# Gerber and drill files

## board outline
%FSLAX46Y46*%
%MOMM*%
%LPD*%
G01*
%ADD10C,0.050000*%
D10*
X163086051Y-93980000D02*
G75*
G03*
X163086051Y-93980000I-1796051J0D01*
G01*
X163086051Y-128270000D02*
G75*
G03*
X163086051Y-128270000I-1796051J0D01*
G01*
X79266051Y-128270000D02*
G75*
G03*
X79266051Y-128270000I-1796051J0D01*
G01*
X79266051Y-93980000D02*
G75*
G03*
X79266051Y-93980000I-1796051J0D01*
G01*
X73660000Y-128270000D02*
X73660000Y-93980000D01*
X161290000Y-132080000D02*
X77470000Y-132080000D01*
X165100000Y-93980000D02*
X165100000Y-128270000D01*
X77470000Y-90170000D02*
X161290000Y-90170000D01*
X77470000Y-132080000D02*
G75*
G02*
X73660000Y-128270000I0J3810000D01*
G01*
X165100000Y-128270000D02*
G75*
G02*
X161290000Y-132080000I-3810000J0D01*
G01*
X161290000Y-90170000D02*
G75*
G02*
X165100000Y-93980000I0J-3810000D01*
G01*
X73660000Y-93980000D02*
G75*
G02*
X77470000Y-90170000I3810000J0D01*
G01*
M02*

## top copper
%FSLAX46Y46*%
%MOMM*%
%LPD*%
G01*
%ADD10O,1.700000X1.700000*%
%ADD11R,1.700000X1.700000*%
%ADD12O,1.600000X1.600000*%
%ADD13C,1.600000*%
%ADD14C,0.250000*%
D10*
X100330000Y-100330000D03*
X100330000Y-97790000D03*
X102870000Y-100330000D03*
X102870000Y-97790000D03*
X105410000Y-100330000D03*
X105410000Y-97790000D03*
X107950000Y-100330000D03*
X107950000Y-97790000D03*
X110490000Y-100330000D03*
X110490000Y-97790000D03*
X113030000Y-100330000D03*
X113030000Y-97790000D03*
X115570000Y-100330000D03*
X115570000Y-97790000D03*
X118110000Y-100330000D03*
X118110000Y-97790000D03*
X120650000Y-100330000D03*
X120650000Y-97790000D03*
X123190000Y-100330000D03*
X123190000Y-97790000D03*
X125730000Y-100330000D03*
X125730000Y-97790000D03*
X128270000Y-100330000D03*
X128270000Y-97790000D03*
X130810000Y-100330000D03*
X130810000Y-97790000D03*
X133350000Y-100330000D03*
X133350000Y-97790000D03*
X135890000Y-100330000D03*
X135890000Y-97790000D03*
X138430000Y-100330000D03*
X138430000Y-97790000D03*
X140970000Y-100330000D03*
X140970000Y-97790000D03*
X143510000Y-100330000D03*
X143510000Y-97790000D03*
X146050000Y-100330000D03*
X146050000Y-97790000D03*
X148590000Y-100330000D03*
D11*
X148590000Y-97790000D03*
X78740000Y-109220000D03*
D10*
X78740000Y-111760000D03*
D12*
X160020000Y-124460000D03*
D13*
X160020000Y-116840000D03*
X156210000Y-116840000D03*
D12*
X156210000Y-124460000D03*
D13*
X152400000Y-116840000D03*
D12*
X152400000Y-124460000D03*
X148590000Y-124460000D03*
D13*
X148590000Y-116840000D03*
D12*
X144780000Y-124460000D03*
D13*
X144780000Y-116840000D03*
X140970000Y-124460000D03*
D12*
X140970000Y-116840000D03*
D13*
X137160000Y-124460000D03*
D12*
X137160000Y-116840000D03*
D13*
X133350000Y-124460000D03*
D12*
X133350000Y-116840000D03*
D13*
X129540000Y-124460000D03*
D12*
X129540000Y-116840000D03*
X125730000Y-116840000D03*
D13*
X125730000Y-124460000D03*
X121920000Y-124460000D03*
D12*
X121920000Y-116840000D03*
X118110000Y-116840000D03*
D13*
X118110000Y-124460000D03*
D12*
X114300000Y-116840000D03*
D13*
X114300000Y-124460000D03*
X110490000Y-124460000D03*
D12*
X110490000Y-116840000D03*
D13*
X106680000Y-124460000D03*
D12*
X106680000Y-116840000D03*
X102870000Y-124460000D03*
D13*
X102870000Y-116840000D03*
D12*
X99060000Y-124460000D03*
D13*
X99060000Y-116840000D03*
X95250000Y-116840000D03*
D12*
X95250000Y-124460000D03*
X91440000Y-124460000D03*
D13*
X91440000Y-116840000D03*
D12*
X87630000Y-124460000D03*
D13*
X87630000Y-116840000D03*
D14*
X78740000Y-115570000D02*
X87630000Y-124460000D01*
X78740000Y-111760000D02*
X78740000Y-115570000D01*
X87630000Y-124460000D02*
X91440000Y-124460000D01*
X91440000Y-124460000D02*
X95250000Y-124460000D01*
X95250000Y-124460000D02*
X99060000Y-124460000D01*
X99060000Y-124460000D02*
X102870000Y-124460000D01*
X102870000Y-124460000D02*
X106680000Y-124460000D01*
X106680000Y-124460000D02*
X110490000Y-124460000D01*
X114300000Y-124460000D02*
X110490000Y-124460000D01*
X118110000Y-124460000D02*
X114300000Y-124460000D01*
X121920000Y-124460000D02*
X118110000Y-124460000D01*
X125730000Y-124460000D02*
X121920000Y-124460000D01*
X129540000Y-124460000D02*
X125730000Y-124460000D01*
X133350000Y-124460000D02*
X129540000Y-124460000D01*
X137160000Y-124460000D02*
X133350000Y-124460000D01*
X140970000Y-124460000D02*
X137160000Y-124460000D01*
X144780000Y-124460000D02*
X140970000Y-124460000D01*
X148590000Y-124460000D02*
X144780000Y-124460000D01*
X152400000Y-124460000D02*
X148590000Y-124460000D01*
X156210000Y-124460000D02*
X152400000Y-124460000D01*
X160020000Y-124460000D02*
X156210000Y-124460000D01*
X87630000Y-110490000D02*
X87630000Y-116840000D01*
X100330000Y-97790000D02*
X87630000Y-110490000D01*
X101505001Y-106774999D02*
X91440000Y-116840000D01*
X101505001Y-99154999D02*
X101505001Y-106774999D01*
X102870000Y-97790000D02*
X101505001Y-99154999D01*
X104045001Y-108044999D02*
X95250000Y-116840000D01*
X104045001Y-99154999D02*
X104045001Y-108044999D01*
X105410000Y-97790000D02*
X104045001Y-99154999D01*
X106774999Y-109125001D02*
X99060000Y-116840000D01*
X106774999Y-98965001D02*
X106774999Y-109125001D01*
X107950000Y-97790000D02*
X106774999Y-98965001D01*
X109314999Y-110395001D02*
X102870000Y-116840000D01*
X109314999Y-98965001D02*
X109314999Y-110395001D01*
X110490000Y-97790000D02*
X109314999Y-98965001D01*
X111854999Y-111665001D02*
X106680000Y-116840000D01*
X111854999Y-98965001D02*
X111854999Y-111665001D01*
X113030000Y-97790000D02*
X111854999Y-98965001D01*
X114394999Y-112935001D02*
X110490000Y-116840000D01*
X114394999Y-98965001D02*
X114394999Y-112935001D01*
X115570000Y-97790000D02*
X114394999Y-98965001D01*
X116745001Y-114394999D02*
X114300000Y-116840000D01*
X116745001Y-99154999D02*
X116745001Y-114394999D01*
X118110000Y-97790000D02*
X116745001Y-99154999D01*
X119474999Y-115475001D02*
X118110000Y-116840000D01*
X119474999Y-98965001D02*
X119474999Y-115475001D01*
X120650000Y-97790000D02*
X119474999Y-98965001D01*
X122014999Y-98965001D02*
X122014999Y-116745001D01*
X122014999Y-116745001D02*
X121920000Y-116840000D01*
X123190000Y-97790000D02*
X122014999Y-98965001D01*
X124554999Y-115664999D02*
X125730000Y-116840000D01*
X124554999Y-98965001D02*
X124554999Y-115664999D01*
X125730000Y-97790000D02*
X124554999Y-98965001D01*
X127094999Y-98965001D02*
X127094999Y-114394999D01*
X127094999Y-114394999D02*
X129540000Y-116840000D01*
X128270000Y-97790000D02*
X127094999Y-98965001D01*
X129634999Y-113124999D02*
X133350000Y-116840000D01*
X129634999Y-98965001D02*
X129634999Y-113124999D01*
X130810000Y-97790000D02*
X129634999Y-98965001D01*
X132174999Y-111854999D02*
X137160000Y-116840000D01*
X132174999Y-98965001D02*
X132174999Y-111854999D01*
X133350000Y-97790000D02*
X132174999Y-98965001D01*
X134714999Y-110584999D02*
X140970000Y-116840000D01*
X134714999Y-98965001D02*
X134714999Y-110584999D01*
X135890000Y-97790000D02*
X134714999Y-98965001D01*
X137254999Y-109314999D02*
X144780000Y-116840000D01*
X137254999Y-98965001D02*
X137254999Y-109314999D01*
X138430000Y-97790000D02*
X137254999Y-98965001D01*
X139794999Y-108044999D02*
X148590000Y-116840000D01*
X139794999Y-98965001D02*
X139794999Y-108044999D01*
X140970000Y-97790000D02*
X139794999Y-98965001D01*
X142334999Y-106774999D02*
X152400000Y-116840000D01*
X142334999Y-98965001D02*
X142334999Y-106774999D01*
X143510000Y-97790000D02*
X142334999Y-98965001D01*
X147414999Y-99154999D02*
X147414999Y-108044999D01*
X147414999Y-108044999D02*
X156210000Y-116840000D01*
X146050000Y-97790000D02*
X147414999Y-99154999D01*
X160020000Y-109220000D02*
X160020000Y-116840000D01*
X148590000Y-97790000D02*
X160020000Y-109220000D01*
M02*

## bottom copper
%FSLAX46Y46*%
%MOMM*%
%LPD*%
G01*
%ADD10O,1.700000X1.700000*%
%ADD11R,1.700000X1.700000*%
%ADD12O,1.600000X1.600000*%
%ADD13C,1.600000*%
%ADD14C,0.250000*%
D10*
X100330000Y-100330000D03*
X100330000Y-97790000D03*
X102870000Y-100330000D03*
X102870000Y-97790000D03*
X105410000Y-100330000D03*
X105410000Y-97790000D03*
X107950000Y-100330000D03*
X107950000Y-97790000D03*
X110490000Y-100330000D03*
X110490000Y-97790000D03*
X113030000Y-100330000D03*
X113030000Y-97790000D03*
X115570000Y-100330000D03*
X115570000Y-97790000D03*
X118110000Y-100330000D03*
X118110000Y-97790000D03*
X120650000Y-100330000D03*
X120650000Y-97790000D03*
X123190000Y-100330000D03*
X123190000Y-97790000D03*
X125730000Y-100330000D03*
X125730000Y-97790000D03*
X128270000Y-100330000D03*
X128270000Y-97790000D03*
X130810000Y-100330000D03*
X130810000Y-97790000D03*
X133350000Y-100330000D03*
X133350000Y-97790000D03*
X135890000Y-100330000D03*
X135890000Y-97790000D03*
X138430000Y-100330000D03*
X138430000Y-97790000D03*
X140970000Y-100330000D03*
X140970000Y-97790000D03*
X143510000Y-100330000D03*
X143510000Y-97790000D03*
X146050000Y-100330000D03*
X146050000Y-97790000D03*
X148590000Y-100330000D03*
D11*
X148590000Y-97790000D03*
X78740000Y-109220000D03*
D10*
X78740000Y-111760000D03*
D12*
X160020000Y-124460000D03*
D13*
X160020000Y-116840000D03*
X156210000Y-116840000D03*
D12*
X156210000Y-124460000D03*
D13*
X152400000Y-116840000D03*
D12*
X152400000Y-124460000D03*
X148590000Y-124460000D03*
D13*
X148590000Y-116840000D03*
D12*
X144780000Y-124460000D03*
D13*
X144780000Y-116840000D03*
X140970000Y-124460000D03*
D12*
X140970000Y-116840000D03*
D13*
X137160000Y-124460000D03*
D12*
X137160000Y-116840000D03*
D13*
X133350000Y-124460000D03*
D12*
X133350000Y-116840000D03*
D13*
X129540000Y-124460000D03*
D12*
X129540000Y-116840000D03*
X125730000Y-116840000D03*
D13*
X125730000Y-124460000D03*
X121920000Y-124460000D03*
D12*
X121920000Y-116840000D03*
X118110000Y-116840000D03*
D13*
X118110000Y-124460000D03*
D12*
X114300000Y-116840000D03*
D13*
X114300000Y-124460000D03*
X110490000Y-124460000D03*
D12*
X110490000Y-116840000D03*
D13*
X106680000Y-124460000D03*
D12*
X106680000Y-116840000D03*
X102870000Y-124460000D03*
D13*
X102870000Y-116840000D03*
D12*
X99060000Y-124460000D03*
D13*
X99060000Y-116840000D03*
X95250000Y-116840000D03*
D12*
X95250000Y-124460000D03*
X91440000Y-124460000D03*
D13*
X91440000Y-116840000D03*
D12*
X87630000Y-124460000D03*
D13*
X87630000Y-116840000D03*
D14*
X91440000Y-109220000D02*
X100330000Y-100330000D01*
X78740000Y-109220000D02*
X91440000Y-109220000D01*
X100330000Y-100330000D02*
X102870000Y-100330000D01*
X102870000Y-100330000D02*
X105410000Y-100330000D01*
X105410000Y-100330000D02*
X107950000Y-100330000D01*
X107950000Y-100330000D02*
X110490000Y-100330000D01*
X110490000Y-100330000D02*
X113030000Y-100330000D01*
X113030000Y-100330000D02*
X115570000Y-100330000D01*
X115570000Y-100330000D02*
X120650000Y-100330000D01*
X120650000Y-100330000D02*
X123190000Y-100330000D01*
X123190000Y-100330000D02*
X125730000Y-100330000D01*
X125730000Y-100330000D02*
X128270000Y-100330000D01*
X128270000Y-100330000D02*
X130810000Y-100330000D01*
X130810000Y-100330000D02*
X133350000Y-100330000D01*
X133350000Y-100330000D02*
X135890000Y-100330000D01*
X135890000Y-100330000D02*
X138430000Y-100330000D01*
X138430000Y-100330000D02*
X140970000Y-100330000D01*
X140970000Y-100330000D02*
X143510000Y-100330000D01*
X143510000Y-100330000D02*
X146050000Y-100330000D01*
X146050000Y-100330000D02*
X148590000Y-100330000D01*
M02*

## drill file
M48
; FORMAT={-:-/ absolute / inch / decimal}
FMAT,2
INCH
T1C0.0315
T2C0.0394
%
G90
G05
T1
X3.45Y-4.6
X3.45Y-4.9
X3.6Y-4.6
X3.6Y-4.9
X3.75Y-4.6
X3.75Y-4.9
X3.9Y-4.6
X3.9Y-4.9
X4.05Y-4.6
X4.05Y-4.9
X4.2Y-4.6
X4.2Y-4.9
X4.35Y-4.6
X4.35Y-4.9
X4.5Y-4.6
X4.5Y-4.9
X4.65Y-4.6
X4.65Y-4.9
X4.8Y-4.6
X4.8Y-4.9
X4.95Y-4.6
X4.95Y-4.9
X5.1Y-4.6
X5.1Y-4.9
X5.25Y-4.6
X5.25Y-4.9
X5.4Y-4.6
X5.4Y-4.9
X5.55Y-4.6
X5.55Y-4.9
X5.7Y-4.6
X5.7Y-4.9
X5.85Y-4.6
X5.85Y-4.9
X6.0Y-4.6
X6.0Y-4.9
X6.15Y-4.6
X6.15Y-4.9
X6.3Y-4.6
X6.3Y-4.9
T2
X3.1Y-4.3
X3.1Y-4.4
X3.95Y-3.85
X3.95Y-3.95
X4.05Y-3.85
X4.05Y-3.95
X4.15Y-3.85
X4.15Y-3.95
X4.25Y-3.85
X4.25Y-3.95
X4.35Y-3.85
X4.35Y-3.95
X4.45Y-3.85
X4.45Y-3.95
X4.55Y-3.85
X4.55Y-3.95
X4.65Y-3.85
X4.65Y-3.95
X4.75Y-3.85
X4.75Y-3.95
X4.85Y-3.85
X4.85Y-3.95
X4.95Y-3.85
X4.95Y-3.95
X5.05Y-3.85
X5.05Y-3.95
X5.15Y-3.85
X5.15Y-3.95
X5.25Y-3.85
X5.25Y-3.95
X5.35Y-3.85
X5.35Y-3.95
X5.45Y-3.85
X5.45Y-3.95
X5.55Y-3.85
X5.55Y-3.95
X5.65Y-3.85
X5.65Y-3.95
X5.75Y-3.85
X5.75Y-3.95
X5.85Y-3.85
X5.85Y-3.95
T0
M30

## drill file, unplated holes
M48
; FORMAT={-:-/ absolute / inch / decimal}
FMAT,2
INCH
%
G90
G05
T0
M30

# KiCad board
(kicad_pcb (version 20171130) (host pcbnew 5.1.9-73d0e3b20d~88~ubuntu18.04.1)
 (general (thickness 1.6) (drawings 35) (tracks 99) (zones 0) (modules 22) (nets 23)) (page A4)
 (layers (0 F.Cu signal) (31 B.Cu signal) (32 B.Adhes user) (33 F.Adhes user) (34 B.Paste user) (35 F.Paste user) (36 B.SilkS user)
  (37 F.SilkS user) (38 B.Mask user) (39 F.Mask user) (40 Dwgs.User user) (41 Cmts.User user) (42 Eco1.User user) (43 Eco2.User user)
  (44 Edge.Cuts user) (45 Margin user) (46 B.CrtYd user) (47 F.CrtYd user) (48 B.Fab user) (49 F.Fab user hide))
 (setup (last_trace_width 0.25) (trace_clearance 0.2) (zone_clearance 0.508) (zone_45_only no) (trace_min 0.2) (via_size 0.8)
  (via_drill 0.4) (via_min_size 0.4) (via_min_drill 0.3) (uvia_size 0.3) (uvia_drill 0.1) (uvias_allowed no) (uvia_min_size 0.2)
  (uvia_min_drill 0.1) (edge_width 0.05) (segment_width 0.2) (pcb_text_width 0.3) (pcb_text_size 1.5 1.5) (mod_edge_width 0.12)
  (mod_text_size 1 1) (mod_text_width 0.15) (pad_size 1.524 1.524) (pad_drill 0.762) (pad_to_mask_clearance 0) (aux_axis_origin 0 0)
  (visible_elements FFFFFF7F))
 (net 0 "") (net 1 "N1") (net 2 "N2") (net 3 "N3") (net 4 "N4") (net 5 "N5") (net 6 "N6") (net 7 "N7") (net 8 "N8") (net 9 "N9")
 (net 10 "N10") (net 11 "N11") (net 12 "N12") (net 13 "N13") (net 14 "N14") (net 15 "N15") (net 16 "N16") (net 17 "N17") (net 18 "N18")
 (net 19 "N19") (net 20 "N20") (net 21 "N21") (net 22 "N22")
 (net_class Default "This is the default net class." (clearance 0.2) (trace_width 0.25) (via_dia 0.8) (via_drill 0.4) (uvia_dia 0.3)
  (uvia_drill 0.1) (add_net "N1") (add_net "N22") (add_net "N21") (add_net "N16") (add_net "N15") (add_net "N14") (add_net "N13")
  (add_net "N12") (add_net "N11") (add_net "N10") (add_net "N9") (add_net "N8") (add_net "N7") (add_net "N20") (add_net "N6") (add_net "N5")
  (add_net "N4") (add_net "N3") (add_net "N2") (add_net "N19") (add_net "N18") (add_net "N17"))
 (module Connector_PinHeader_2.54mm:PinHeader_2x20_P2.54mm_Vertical (layer F.Cu) (at 148.59 97.79 270)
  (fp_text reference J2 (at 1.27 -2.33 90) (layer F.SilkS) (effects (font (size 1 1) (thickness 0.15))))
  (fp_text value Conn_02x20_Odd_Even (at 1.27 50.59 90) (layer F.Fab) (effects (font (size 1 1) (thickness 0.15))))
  (pad 40 thru_hole oval (at 2.54 48.26 270) (size 1.7 1.7) (drill 1) (layers *.Cu *.Mask) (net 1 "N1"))
  (pad 39 thru_hole oval (at 0 48.26 270) (size 1.7 1.7) (drill 1) (layers *.Cu *.Mask) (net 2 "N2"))
  (pad 38 thru_hole oval (at 2.54 45.72 270) (size 1.7 1.7) (drill 1) (layers *.Cu *.Mask) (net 1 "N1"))
  (pad 37 thru_hole oval (at 0 45.72 270) (size 1.7 1.7) (drill 1) (layers *.Cu *.Mask) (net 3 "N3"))
  (pad 36 thru_hole oval (at 2.54 43.18 270) (size 1.7 1.7) (drill 1) (layers *.Cu *.Mask) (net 1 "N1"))
  (pad 35 thru_hole oval (at 0 43.18 270) (size 1.7 1.7) (drill 1) (layers *.Cu *.Mask) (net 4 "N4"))
  (pad 34 thru_hole oval (at 2.54 40.64 270) (size 1.7 1.7) (drill 1) (layers *.Cu *.Mask) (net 1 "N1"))
  (pad 33 thru_hole oval (at 0 40.64 270) (size 1.7 1.7) (drill 1) (layers *.Cu *.Mask) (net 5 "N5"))
  (pad 32 thru_hole oval (at 2.54 38.1 270) (size 1.7 1.7) (drill 1) (layers *.Cu *.Mask) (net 1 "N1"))
  (pad 31 thru_hole oval (at 0 38.1 270) (size 1.7 1.7) (drill 1) (layers *.Cu *.Mask) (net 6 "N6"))
  (pad 30 thru_hole oval (at 2.54 35.56 270) (size 1.7 1.7) (drill 1) (layers *.Cu *.Mask) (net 1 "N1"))
  (pad 29 thru_hole oval (at 0 35.56 270) (size 1.7 1.7) (drill 1) (layers *.Cu *.Mask) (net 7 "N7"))
  (pad 28 thru_hole oval (at 2.54 33.02 270) (size 1.7 1.7) (drill 1) (layers *.Cu *.Mask) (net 1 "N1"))
  (pad 27 thru_hole oval (at 0 33.02 270) (size 1.7 1.7) (drill 1) (layers *.Cu *.Mask) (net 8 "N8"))
  (pad 26 thru_hole oval (at 2.54 30.48 270) (size 1.7 1.7) (drill 1) (layers *.Cu *.Mask) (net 1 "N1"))
  (pad 25 thru_hole oval (at 0 30.48 270) (size 1.7 1.7) (drill 1) (layers *.Cu *.Mask) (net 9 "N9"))
  (pad 24 thru_hole oval (at 2.54 27.94 270) (size 1.7 1.7) (drill 1) (layers *.Cu *.Mask) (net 1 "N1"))
  (pad 23 thru_hole oval (at 0 27.94 270) (size 1.7 1.7) (drill 1) (layers *.Cu *.Mask) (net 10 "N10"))
  (pad 22 thru_hole oval (at 2.54 25.4 270) (size 1.7 1.7) (drill 1) (layers *.Cu *.Mask) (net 1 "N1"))
  (pad 21 thru_hole oval (at 0 25.4 270) (size 1.7 1.7) (drill 1) (layers *.Cu *.Mask) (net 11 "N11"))
  (pad 20 thru_hole oval (at 2.54 22.86 270) (size 1.7 1.7) (drill 1) (layers *.Cu *.Mask) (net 1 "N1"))
  (pad 19 thru_hole oval (at 0 22.86 270) (size 1.7 1.7) (drill 1) (layers *.Cu *.Mask) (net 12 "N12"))
  (pad 18 thru_hole oval (at 2.54 20.32 270) (size 1.7 1.7) (drill 1) (layers *.Cu *.Mask) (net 1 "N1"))
  (pad 17 thru_hole oval (at 0 20.32 270) (size 1.7 1.7) (drill 1) (layers *.Cu *.Mask) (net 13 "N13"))
  (pad 16 thru_hole oval (at 2.54 17.78 270) (size 1.7 1.7) (drill 1) (layers *.Cu *.Mask) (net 1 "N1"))
  (pad 15 thru_hole oval (at 0 17.78 270) (size 1.7 1.7) (drill 1) (layers *.Cu *.Mask) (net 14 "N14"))
  (pad 14 thru_hole oval (at 2.54 15.24 270) (size 1.7 1.7) (drill 1) (layers *.Cu *.Mask) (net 1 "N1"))
  (pad 13 thru_hole oval (at 0 15.24 270) (size 1.7 1.7) (drill 1) (layers *.Cu *.Mask) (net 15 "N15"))
  (pad 12 thru_hole oval (at 2.54 12.7 270) (size 1.7 1.7) (drill 1) (layers *.Cu *.Mask) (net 1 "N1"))
  (pad 11 thru_hole oval (at 0 12.7 270) (size 1.7 1.7) (drill 1) (layers *.Cu *.Mask) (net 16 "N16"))
  (pad 10 thru_hole oval (at 2.54 10.16 270) (size 1.7 1.7) (drill 1) (layers *.Cu *.Mask) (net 1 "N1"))
  (pad 9 thru_hole oval (at 0 10.16 270) (size 1.7 1.7) (drill 1) (layers *.Cu *.Mask) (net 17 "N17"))
  (pad 8 thru_hole oval (at 2.54 7.62 270) (size 1.7 1.7) (drill 1) (layers *.Cu *.Mask) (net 1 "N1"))
  (pad 7 thru_hole oval (at 0 7.62 270) (size 1.7 1.7) (drill 1) (layers *.Cu *.Mask) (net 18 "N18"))
  (pad 6 thru_hole oval (at 2.54 5.08 270) (size 1.7 1.7) (drill 1) (layers *.Cu *.Mask) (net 1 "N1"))
  (pad 5 thru_hole oval (at 0 5.08 270) (size 1.7 1.7) (drill 1) (layers *.Cu *.Mask) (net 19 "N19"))
  (pad 4 thru_hole oval (at 2.54 2.54 270) (size 1.7 1.7) (drill 1) (layers *.Cu *.Mask) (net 1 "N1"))
  (pad 3 thru_hole oval (at 0 2.54 270) (size 1.7 1.7) (drill 1) (layers *.Cu *.Mask) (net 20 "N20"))
  (pad 2 thru_hole oval (at 2.54 0 270) (size 1.7 1.7) (drill 1) (layers *.Cu *.Mask) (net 1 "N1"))
  (pad 1 thru_hole rect (at 0 0 270) (size 1.7 1.7) (drill 1) (layers *.Cu *.Mask) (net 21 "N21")))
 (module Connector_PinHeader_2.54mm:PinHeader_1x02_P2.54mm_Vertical (layer F.Cu) (at 78.74 109.22)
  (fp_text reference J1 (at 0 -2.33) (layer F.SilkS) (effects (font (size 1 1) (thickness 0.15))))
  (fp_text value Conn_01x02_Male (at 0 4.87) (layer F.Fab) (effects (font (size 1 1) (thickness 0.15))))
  (pad 1 thru_hole rect (at 0 0) (size 1.7 1.7) (drill 1) (layers *.Cu *.Mask) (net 1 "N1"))
  (pad 2 thru_hole oval (at 0 2.54) (size 1.7 1.7) (drill 1) (layers *.Cu *.Mask) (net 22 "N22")))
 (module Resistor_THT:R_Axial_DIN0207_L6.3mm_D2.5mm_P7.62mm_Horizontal (layer F.Cu) (at 160.02 116.84 270)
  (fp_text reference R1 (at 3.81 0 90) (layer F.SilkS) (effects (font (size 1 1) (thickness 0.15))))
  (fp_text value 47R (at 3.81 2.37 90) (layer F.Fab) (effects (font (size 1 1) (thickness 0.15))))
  (pad 2 thru_hole oval (at 7.62 0 270) (size 1.6 1.6) (drill 0.8) (layers *.Cu *.Mask) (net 22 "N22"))
  (pad 1 thru_hole circle (at 0 0 270) (size 1.6 1.6) (drill 0.8) (layers *.Cu *.Mask) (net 21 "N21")))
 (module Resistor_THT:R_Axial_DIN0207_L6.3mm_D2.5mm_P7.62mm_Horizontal (layer F.Cu) (at 156.21 116.84 270)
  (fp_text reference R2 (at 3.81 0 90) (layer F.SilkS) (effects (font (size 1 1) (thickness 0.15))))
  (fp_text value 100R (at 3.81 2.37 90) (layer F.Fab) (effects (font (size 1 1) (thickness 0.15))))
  (pad 1 thru_hole circle (at 0 0 270) (size 1.6 1.6) (drill 0.8) (layers *.Cu *.Mask) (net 20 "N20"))
  (pad 2 thru_hole oval (at 7.62 0 270) (size 1.6 1.6) (drill 0.8) (layers *.Cu *.Mask) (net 22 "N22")))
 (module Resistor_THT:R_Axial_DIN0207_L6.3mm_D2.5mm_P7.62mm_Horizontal (layer F.Cu) (at 152.4 116.84 270)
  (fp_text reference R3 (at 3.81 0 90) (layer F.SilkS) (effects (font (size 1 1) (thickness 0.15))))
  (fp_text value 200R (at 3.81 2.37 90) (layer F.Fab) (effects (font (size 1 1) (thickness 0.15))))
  (pad 1 thru_hole circle (at 0 0 270) (size 1.6 1.6) (drill 0.8) (layers *.Cu *.Mask) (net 19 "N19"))
  (pad 2 thru_hole oval (at 7.62 0 270) (size 1.6 1.6) (drill 0.8) (layers *.Cu *.Mask) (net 22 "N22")))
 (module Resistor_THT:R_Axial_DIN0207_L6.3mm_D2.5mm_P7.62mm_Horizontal (layer F.Cu) (at 148.59 116.84 270)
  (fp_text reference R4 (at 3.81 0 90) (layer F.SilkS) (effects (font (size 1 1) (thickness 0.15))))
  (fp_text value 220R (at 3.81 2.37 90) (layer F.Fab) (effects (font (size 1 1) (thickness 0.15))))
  (pad 2 thru_hole oval (at 7.62 0 270) (size 1.6 1.6) (drill 0.8) (layers *.Cu *.Mask) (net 22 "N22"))
  (pad 1 thru_hole circle (at 0 0 270) (size 1.6 1.6) (drill 0.8) (layers *.Cu *.Mask) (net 18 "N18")))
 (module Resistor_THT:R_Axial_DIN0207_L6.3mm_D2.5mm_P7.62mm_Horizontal (layer F.Cu) (at 144.78 116.84 270)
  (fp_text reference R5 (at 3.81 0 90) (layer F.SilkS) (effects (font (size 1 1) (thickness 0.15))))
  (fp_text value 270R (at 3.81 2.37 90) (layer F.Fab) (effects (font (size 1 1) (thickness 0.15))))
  (pad 2 thru_hole oval (at 7.62 0 270) (size 1.6 1.6) (drill 0.8) (layers *.Cu *.Mask) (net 22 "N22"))
  (pad 1 thru_hole circle (at 0 0 270) (size 1.6 1.6) (drill 0.8) (layers *.Cu *.Mask) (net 17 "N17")))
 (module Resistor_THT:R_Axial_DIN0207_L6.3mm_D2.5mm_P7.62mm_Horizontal (layer F.Cu) (at 140.97 124.46 90)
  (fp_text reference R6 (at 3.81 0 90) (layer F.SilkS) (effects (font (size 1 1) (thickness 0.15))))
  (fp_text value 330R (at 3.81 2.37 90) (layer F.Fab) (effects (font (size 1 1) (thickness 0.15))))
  (pad 1 thru_hole circle (at 0 0 90) (size 1.6 1.6) (drill 0.8) (layers *.Cu *.Mask) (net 22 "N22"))
  (pad 2 thru_hole oval (at 7.62 0 90) (size 1.6 1.6) (drill 0.8) (layers *.Cu *.Mask) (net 16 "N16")))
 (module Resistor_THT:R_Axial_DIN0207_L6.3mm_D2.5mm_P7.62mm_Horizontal (layer F.Cu) (at 137.16 124.46 90)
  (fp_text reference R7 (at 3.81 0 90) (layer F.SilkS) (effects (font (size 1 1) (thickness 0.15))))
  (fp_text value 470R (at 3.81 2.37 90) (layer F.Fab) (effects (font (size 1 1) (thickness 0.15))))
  (pad 1 thru_hole circle (at 0 0 90) (size 1.6 1.6) (drill 0.8) (layers *.Cu *.Mask) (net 22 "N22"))
  (pad 2 thru_hole oval (at 7.62 0 90) (size 1.6 1.6) (drill 0.8) (layers *.Cu *.Mask) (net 15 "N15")))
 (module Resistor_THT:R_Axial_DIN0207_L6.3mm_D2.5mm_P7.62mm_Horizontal (layer F.Cu) (at 133.35 124.46 90)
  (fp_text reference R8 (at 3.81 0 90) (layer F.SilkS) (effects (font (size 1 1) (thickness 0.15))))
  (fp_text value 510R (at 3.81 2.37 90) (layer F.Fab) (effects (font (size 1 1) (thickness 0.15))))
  (pad 1 thru_hole circle (at 0 0 90) (size 1.6 1.6) (drill 0.8) (layers *.Cu *.Mask) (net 22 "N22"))
  (pad 2 thru_hole oval (at 7.62 0 90) (size 1.6 1.6) (drill 0.8) (layers *.Cu *.Mask) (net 14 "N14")))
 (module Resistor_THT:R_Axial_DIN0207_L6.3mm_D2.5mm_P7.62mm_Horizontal (layer F.Cu) (at 129.54 124.46 90)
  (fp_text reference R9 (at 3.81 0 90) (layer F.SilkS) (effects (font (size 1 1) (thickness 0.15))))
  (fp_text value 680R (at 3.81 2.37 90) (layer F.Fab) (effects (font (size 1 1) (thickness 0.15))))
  (pad 1 thru_hole circle (at 0 0 90) (size 1.6 1.6) (drill 0.8) (layers *.Cu *.Mask) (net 22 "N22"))
  (pad 2 thru_hole oval (at 7.62 0 90) (size 1.6 1.6) (drill 0.8) (layers *.Cu *.Mask) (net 13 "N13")))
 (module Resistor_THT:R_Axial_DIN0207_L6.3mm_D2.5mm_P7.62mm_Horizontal (layer F.Cu) (at 125.73 124.46 90)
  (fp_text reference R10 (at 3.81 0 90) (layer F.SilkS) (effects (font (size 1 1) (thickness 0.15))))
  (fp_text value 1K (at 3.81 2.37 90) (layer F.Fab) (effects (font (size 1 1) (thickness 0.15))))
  (pad 2 thru_hole oval (at 7.62 0 90) (size 1.6 1.6) (drill 0.8) (layers *.Cu *.Mask) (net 12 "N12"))
  (pad 1 thru_hole circle (at 0 0 90) (size 1.6 1.6) (drill 0.8) (layers *.Cu *.Mask) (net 22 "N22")))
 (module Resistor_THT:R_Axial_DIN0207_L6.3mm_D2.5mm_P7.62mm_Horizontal (layer F.Cu) (at 121.92 124.46 90)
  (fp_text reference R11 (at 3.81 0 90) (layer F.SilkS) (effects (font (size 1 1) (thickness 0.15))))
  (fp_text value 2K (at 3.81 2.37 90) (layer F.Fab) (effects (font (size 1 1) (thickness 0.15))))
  (pad 1 thru_hole circle (at 0 0 90) (size 1.6 1.6) (drill 0.8) (layers *.Cu *.Mask) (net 22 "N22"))
  (pad 2 thru_hole oval (at 7.62 0 90) (size 1.6 1.6) (drill 0.8) (layers *.Cu *.Mask) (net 11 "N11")))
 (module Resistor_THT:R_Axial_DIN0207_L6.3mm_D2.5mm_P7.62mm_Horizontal (layer F.Cu) (at 118.11 124.46 90)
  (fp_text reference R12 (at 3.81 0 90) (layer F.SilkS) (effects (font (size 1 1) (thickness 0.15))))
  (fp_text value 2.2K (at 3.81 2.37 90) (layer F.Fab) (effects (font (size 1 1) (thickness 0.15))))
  (pad 2 thru_hole oval (at 7.62 0 90) (size 1.6 1.6) (drill 0.8) (layers *.Cu *.Mask) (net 10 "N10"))
  (pad 1 thru_hole circle (at 0 0 90) (size 1.6 1.6) (drill 0.8) (layers *.Cu *.Mask) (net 22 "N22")))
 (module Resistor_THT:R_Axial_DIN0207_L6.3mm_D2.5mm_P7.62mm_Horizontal (layer F.Cu) (at 114.3 124.46 90)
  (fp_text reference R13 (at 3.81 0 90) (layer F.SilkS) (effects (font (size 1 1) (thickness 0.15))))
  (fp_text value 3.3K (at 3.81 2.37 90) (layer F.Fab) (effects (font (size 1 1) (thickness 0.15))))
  (pad 2 thru_hole oval (at 7.62 0 90) (size 1.6 1.6) (drill 0.8) (layers *.Cu *.Mask) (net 9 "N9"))
  (pad 1 thru_hole circle (at 0 0 90) (size 1.6 1.6) (drill 0.8) (layers *.Cu *.Mask) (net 22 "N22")))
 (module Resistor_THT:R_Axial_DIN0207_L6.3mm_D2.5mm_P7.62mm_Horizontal (layer F.Cu) (at 110.49 124.46 90)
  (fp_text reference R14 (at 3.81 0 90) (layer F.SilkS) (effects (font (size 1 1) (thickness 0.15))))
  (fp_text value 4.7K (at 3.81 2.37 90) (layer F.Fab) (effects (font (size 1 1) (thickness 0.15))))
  (pad 1 thru_hole circle (at 0 0 90) (size 1.6 1.6) (drill 0.8) (layers *.Cu *.Mask) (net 22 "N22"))
  (pad 2 thru_hole oval (at 7.62 0 90) (size 1.6 1.6) (drill 0.8) (layers *.Cu *.Mask) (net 8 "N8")))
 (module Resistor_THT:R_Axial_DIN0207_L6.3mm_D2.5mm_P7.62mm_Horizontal (layer F.Cu) (at 106.68 124.46 90)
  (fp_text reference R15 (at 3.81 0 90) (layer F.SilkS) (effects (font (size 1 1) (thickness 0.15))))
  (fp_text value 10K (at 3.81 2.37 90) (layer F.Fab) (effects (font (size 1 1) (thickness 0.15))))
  (pad 1 thru_hole circle (at 0 0 90) (size 1.6 1.6) (drill 0.8) (layers *.Cu *.Mask) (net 22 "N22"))
  (pad 2 thru_hole oval (at 7.62 0 90) (size 1.6 1.6) (drill 0.8) (layers *.Cu *.Mask) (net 7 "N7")))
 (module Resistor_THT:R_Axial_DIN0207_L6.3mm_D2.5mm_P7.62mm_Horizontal (layer F.Cu) (at 102.87 116.84 270)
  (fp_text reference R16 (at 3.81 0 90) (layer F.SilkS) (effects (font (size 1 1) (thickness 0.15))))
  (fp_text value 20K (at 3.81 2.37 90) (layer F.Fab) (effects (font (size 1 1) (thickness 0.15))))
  (pad 2 thru_hole oval (at 7.62 0 270) (size 1.6 1.6) (drill 0.8) (layers *.Cu *.Mask) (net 22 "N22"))
  (pad 1 thru_hole circle (at 0 0 270) (size 1.6 1.6) (drill 0.8) (layers *.Cu *.Mask) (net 6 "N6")))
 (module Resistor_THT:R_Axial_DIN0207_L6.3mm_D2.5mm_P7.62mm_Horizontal (layer F.Cu) (at 99.06 116.84 270)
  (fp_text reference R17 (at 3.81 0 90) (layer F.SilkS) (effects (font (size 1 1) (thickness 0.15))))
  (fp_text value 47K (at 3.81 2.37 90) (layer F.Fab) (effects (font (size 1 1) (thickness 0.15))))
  (pad 2 thru_hole oval (at 7.62 0 270) (size 1.6 1.6) (drill 0.8) (layers *.Cu *.Mask) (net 22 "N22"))
  (pad 1 thru_hole circle (at 0 0 270) (size 1.6 1.6) (drill 0.8) (layers *.Cu *.Mask) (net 5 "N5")))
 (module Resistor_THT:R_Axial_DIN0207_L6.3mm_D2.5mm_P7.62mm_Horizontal (layer F.Cu) (at 95.25 116.84 270)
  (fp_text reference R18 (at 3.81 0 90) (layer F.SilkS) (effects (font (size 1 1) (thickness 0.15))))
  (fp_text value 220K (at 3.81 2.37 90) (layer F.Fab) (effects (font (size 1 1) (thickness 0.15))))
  (pad 1 thru_hole circle (at 0 0 270) (size 1.6 1.6) (drill 0.8) (layers *.Cu *.Mask) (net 4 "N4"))
  (pad 2 thru_hole oval (at 7.62 0 270) (size 1.6 1.6) (drill 0.8) (layers *.Cu *.Mask) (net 22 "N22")))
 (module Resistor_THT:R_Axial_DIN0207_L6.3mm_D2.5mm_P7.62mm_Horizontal (layer F.Cu) (at 91.44 116.84 270)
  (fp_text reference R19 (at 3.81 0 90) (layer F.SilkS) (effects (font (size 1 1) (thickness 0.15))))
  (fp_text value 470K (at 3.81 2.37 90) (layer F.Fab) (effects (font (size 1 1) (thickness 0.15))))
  (pad 2 thru_hole oval (at 7.62 0 270) (size 1.6 1.6) (drill 0.8) (layers *.Cu *.Mask) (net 22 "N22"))
  (pad 1 thru_hole circle (at 0 0 270) (size 1.6 1.6) (drill 0.8) (layers *.Cu *.Mask) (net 3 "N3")))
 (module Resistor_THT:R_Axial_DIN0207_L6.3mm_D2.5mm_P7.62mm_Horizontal (layer F.Cu) (at 87.63 116.84 270)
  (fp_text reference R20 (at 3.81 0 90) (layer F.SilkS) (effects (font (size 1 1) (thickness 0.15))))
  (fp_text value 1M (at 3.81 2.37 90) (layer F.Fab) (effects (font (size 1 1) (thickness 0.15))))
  (pad 2 thru_hole oval (at 7.62 0 270) (size 1.6 1.6) (drill 0.8) (layers *.Cu *.Mask) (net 22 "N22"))
  (pad 1 thru_hole circle (at 0 0 270) (size 1.6 1.6) (drill 0.8) (layers *.Cu *.Mask) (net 2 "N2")))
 (gr_circle (center 161.29 93.98) (end 162.56 92.71) (layer Edge.Cuts) (width 0.05))
 (gr_circle (center 161.29 128.27) (end 162.56 129.54) (layer Edge.Cuts) (width 0.05))
 (gr_circle (center 77.47 128.27) (end 76.2 129.54) (layer Edge.Cuts) (width 0.05))
 (gr_circle (center 77.47 93.98) (end 76.2 92.71) (layer Edge.Cuts) (width 0.05))
 (gr_line (start 73.66 128.27) (end 73.66 93.98) (layer Edge.Cuts) (width 0.05))
 (gr_line (start 161.29 132.08) (end 77.47 132.08) (layer Edge.Cuts) (width 0.05))
 (gr_line (start 165.1 93.98) (end 165.1 128.27) (layer Edge.Cuts) (width 0.05))
 (gr_line (start 77.47 90.17) (end 161.29 90.17) (layer Edge.Cuts) (width 0.05))
 (gr_arc (start 77.47 128.27) (end 73.66 128.27) (angle -90) (layer Edge.Cuts) (width 0.05))
 (gr_arc (start 161.29 128.27) (end 161.29 132.08) (angle -90) (layer Edge.Cuts) (width 0.05))
 (gr_arc (start 161.29 93.98) (end 165.1 93.98) (angle -90) (layer Edge.Cuts) (width 0.05))
 (gr_arc (start 77.47 93.98) (end 77.47 90.17) (angle -90) (layer Edge.Cuts) (width 0.05))
 (segment (start 91.44 109.22) (end 100.33 100.33) (width 0.25) (layer B.Cu) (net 1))
 (segment (start 78.74 109.22) (end 91.44 109.22) (width 0.25) (layer B.Cu) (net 1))
 (segment (start 100.33 100.33) (end 102.87 100.33) (width 0.25) (layer B.Cu) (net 1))
 (segment (start 102.87 100.33) (end 105.41 100.33) (width 0.25) (layer B.Cu) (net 1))
 (segment (start 105.41 100.33) (end 107.95 100.33) (width 0.25) (layer B.Cu) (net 1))
 (segment (start 107.95 100.33) (end 110.49 100.33) (width 0.25) (layer B.Cu) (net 1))
 (segment (start 110.49 100.33) (end 113.03 100.33) (width 0.25) (layer B.Cu) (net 1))
 (segment (start 113.03 100.33) (end 115.57 100.33) (width 0.25) (layer B.Cu) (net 1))
 (segment (start 115.57 100.33) (end 120.65 100.33) (width 0.25) (layer B.Cu) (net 1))
 (segment (start 120.65 100.33) (end 123.19 100.33) (width 0.25) (layer B.Cu) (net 1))
 (segment (start 123.19 100.33) (end 125.73 100.33) (width 0.25) (layer B.Cu) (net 1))
 (segment (start 125.73 100.33) (end 128.27 100.33) (width 0.25) (layer B.Cu) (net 1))
 (segment (start 128.27 100.33) (end 130.81 100.33) (width 0.25) (layer B.Cu) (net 1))
 (segment (start 130.81 100.33) (end 133.35 100.33) (width 0.25) (layer B.Cu) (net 1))
 (segment (start 133.35 100.33) (end 135.89 100.33) (width 0.25) (layer B.Cu) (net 1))
 (segment (start 135.89 100.33) (end 138.43 100.33) (width 0.25) (layer B.Cu) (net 1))
 (segment (start 138.43 100.33) (end 140.97 100.33) (width 0.25) (layer B.Cu) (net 1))
 (segment (start 140.97 100.33) (end 143.51 100.33) (width 0.25) (layer B.Cu) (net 1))
 (segment (start 143.51 100.33) (end 146.05 100.33) (width 0.25) (layer B.Cu) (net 1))
 (segment (start 146.05 100.33) (end 148.59 100.33) (width 0.25) (layer B.Cu) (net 1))
 (segment (start 78.74 115.57) (end 87.63 124.46) (width 0.25) (layer F.Cu) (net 22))
 (segment (start 78.74 111.76) (end 78.74 115.57) (width 0.25) (layer F.Cu) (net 22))
 (segment (start 87.63 124.46) (end 91.44 124.46) (width 0.25) (layer F.Cu) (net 22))
 (segment (start 91.44 124.46) (end 95.25 124.46) (width 0.25) (layer F.Cu) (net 22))
 (segment (start 95.25 124.46) (end 99.06 124.46) (width 0.25) (layer F.Cu) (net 22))
 (segment (start 99.06 124.46) (end 102.87 124.46) (width 0.25) (layer F.Cu) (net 22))
 (segment (start 102.87 124.46) (end 106.68 124.46) (width 0.25) (layer F.Cu) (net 22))
 (segment (start 106.68 124.46) (end 110.49 124.46) (width 0.25) (layer F.Cu) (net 22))
 (segment (start 114.3 124.46) (end 110.49 124.46) (width 0.25) (layer F.Cu) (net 22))
 (segment (start 118.11 124.46) (end 114.3 124.46) (width 0.25) (layer F.Cu) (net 22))
 (segment (start 121.92 124.46) (end 118.11 124.46) (width 0.25) (layer F.Cu) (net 22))
 (segment (start 125.73 124.46) (end 121.92 124.46) (width 0.25) (layer F.Cu) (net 22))
 (segment (start 129.54 124.46) (end 125.73 124.46) (width 0.25) (layer F.Cu) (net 22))
 (segment (start 133.35 124.46) (end 129.54 124.46) (width 0.25) (layer F.Cu) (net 22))
 (segment (start 137.16 124.46) (end 133.35 124.46) (width 0.25) (layer F.Cu) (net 22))
 (segment (start 140.97 124.46) (end 137.16 124.46) (width 0.25) (layer F.Cu) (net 22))
 (segment (start 144.78 124.46) (end 140.97 124.46) (width 0.25) (layer F.Cu) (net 22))
 (segment (start 148.59 124.46) (end 144.78 124.46) (width 0.25) (layer F.Cu) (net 22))
 (segment (start 152.4 124.46) (end 148.59 124.46) (width 0.25) (layer F.Cu) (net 22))
 (segment (start 156.21 124.46) (end 152.4 124.46) (width 0.25) (layer F.Cu) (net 22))
 (segment (start 160.02 124.46) (end 156.21 124.46) (width 0.25) (layer F.Cu) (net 22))
 (segment (start 87.63 110.49) (end 87.63 116.84) (width 0.25) (layer F.Cu) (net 2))
 (segment (start 100.33 97.79) (end 87.63 110.49) (width 0.25) (layer F.Cu) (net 2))
 (segment (start 101.505001 106.774999) (end 91.44 116.84) (width 0.25) (layer F.Cu) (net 3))
 (segment (start 101.505001 99.154999) (end 101.505001 106.774999) (width 0.25) (layer F.Cu) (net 3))
 (segment (start 102.87 97.79) (end 101.505001 99.154999) (width 0.25) (layer F.Cu) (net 3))
 (segment (start 104.045001 108.044999) (end 95.25 116.84) (width 0.25) (layer F.Cu) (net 4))
 (segment (start 104.045001 99.154999) (end 104.045001 108.044999) (width 0.25) (layer F.Cu) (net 4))
 (segment (start 105.41 97.79) (end 104.045001 99.154999) (width 0.25) (layer F.Cu) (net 4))
 (segment (start 106.774999 109.125001) (end 99.06 116.84) (width 0.25) (layer F.Cu) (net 5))
 (segment (start 106.774999 98.965001) (end 106.774999 109.125001) (width 0.25) (layer F.Cu) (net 5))
 (segment (start 107.95 97.79) (end 106.774999 98.965001) (width 0.25) (layer F.Cu) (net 5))
 (segment (start 109.314999 110.395001) (end 102.87 116.84) (width 0.25) (layer F.Cu) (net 6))
 (segment (start 109.314999 98.965001) (end 109.314999 110.395001) (width 0.25) (layer F.Cu) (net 6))
 (segment (start 110.49 97.79) (end 109.314999 98.965001) (width 0.25) (layer F.Cu) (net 6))
 (segment (start 111.854999 111.665001) (end 106.68 116.84) (width 0.25) (layer F.Cu) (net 7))
 (segment (start 111.854999 98.965001) (end 111.854999 111.665001) (width 0.25) (layer F.Cu) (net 7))
 (segment (start 113.03 97.79) (end 111.854999 98.965001) (width 0.25) (layer F.Cu) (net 7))
 (segment (start 114.394999 112.935001) (end 110.49 116.84) (width 0.25) (layer F.Cu) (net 8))
 (segment (start 114.394999 98.965001) (end 114.394999 112.935001) (width 0.25) (layer F.Cu) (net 8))
 (segment (start 115.57 97.79) (end 114.394999 98.965001) (width 0.25) (layer F.Cu) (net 8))
 (segment (start 116.745001 114.394999) (end 114.3 116.84) (width 0.25) (layer F.Cu) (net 9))
 (segment (start 116.745001 99.154999) (end 116.745001 114.394999) (width 0.25) (layer F.Cu) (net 9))
 (segment (start 118.11 97.79) (end 116.745001 99.154999) (width 0.25) (layer F.Cu) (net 9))
 (segment (start 119.474999 115.475001) (end 118.11 116.84) (width 0.25) (layer F.Cu) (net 10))
 (segment (start 119.474999 98.965001) (end 119.474999 115.475001) (width 0.25) (layer F.Cu) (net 10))
 (segment (start 120.65 97.79) (end 119.474999 98.965001) (width 0.25) (layer F.Cu) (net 10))
 (segment (start 122.014999 98.965001) (end 122.014999 116.745001) (width 0.25) (layer F.Cu) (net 11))
 (segment (start 122.014999 116.745001) (end 121.92 116.84) (width 0.25) (layer F.Cu) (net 11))
 (segment (start 123.19 97.79) (end 122.014999 98.965001) (width 0.25) (layer F.Cu) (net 11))
 (segment (start 124.554999 115.664999) (end 125.73 116.84) (width 0.25) (layer F.Cu) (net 12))
 (segment (start 124.554999 98.965001) (end 124.554999 115.664999) (width 0.25) (layer F.Cu) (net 12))
 (segment (start 125.73 97.79) (end 124.554999 98.965001) (width 0.25) (layer F.Cu) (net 12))
 (segment (start 127.094999 98.965001) (end 127.094999 114.394999) (width 0.25) (layer F.Cu) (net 13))
 (segment (start 127.094999 114.394999) (end 129.54 116.84) (width 0.25) (layer F.Cu) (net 13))
 (segment (start 128.27 97.79) (end 127.094999 98.965001) (width 0.25) (layer F.Cu) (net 13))
 (segment (start 129.634999 113.124999) (end 133.35 116.84) (width 0.25) (layer F.Cu) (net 14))
 (segment (start 129.634999 98.965001) (end 129.634999 113.124999) (width 0.25) (layer F.Cu) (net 14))
 (segment (start 130.81 97.79) (end 129.634999 98.965001) (width 0.25) (layer F.Cu) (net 14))
 (segment (start 132.174999 111.854999) (end 137.16 116.84) (width 0.25) (layer F.Cu) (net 15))
 (segment (start 132.174999 98.965001) (end 132.174999 111.854999) (width 0.25) (layer F.Cu) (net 15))
 (segment (start 133.35 97.79) (end 132.174999 98.965001) (width 0.25) (layer F.Cu) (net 15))
 (segment (start 134.714999 110.584999) (end 140.97 116.84) (width 0.25) (layer F.Cu) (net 16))
 (segment (start 134.714999 98.965001) (end 134.714999 110.584999) (width 0.25) (layer F.Cu) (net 16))
 (segment (start 135.89 97.79) (end 134.714999 98.965001) (width 0.25) (layer F.Cu) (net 16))
 (segment (start 137.254999 109.314999) (end 144.78 116.84) (width 0.25) (layer F.Cu) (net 17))
 (segment (start 137.254999 98.965001) (end 137.254999 109.314999) (width 0.25) (layer F.Cu) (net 17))
 (segment (start 138.43 97.79) (end 137.254999 98.965001) (width 0.25) (layer F.Cu) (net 17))
 (segment (start 139.794999 108.044999) (end 148.59 116.84) (width 0.25) (layer F.Cu) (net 18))
 (segment (start 139.794999 98.965001) (end 139.794999 108.044999) (width 0.25) (layer F.Cu) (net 18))
 (segment (start 140.97 97.79) (end 139.794999 98.965001) (width 0.25) (layer F.Cu) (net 18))
 (segment (start 142.334999 106.774999) (end 152.4 116.84) (width 0.25) (layer F.Cu) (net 19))
 (segment (start 142.334999 98.965001) (end 142.334999 106.774999) (width 0.25) (layer F.Cu) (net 19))
 (segment (start 143.51 97.79) (end 142.334999 98.965001) (width 0.25) (layer F.Cu) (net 19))
 (segment (start 147.414999 99.154999) (end 147.414999 108.044999) (width 0.25) (layer F.Cu) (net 20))
 (segment (start 147.414999 108.044999) (end 156.21 116.84) (width 0.25) (layer F.Cu) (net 20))
 (segment (start 146.05 97.79) (end 147.414999 99.154999) (width 0.25) (layer F.Cu) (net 20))
 (segment (start 160.02 109.22) (end 160.02 116.84) (width 0.25) (layer F.Cu) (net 21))
 (segment (start 148.59 97.79) (end 160.02 109.22) (width 0.25) (layer F.Cu) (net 21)))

